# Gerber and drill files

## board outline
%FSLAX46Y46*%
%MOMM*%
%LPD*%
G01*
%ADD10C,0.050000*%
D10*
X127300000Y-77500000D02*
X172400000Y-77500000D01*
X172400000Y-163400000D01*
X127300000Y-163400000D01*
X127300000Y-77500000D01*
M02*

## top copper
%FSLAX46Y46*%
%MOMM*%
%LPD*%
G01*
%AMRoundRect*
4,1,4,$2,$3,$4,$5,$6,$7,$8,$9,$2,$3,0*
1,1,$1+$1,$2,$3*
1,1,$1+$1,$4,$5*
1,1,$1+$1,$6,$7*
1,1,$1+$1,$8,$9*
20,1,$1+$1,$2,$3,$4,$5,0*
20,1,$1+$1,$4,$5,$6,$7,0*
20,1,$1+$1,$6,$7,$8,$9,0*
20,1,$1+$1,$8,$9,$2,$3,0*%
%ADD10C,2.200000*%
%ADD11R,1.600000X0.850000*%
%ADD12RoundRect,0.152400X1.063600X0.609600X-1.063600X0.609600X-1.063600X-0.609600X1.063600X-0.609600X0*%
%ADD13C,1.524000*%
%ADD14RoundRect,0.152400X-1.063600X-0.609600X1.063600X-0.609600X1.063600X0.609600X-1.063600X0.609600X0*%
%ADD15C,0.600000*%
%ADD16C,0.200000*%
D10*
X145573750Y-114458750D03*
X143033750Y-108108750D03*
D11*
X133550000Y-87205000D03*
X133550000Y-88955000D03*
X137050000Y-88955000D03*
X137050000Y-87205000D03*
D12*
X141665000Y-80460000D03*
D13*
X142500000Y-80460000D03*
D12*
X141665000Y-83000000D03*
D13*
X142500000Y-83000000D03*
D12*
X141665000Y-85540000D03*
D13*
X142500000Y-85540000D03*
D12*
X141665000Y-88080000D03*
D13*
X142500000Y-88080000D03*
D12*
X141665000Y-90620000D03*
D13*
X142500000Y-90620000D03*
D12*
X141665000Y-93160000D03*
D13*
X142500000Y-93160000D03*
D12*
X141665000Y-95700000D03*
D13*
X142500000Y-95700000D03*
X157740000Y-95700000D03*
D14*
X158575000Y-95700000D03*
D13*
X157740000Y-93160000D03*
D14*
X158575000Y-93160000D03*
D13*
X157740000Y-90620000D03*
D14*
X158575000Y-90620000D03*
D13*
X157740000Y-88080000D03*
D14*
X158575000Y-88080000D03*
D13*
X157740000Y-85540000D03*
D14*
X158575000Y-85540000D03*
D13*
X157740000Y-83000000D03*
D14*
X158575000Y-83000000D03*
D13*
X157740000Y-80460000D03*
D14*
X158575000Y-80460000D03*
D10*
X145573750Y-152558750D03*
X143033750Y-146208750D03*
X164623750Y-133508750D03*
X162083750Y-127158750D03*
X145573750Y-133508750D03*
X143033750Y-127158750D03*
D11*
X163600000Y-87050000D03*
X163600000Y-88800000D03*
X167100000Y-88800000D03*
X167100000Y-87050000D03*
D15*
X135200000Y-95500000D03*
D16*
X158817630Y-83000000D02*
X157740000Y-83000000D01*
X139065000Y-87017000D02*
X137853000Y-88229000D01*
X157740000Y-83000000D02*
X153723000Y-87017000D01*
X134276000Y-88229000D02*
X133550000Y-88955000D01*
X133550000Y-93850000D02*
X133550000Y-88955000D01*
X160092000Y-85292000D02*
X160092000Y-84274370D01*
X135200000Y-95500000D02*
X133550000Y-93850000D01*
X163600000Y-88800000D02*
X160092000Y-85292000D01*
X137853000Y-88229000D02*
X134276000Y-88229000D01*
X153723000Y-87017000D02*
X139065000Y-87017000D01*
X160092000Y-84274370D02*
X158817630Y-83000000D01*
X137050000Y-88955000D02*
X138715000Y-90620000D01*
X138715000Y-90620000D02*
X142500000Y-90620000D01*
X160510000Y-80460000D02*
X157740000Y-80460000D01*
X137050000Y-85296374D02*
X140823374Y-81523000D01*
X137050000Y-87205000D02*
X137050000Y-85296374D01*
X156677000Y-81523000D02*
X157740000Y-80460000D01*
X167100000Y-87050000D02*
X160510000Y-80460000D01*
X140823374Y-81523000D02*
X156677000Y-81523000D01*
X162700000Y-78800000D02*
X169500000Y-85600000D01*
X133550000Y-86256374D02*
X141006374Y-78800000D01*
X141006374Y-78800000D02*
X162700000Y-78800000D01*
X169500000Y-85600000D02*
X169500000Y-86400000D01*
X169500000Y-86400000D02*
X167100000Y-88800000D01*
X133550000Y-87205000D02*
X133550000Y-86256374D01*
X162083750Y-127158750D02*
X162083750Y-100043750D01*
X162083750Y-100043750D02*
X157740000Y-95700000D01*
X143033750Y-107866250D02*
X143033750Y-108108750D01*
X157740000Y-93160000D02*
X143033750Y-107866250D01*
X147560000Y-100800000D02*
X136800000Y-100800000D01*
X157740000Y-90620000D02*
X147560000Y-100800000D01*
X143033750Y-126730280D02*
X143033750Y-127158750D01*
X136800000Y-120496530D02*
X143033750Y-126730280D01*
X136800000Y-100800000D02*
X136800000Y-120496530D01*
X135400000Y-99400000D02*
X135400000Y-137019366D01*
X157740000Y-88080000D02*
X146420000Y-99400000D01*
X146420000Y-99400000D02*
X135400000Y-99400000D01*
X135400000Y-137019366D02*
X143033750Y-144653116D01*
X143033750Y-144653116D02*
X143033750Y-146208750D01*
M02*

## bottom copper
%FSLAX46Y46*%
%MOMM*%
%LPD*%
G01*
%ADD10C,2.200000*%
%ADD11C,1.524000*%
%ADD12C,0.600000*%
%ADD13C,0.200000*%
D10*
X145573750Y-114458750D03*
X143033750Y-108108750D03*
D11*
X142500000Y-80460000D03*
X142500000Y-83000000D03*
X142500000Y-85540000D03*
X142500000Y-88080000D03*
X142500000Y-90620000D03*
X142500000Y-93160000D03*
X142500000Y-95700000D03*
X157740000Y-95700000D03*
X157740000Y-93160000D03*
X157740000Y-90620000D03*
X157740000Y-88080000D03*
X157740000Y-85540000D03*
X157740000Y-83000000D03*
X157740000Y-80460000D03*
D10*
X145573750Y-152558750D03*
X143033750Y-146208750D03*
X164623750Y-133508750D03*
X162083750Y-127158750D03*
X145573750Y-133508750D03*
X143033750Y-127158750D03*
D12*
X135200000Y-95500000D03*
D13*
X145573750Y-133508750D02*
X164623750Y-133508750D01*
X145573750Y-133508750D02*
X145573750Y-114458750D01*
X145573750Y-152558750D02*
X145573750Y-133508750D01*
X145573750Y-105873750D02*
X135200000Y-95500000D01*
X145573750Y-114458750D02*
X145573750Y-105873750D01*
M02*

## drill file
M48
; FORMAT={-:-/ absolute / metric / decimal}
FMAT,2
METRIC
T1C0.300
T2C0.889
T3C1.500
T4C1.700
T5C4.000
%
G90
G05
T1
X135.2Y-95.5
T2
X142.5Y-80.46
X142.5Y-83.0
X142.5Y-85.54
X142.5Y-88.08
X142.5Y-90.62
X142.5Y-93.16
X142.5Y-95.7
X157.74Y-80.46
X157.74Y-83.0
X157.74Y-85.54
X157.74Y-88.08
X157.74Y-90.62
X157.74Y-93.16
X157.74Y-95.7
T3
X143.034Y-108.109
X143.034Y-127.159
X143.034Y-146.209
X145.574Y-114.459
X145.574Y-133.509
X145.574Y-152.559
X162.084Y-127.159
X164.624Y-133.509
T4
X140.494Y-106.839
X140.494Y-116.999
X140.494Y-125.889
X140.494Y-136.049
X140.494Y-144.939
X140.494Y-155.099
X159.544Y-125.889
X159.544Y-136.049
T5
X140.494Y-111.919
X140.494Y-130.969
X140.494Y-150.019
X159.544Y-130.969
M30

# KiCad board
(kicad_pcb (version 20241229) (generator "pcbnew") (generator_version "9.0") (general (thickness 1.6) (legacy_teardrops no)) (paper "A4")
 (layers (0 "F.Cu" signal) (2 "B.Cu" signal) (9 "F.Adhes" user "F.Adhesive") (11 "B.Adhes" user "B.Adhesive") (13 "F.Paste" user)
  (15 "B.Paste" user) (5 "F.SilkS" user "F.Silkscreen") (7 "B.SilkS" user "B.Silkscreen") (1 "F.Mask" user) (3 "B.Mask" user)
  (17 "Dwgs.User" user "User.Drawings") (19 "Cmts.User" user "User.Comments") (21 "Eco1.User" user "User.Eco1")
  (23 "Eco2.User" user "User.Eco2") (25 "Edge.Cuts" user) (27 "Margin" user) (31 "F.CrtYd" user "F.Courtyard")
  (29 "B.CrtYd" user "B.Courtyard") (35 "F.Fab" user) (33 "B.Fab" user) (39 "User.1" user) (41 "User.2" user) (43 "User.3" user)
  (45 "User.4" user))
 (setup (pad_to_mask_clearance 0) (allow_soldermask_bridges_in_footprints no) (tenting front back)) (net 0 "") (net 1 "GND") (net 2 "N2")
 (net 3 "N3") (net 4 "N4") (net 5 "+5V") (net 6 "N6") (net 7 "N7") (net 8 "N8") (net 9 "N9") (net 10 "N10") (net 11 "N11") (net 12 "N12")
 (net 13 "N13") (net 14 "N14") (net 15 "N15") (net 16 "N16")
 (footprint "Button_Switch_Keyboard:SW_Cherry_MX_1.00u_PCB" (layer "F.Cu") (at 145.57375 114.45875 -90)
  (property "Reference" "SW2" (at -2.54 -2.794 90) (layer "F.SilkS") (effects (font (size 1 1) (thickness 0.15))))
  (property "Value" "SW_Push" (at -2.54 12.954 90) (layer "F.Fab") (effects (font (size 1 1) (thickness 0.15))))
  (pad "" np_thru_hole circle (at -7.62 5.08 270) (size 1.7 1.7) (drill 1.7) (layers "*.Cu" "*.Mask"))
  (pad "" np_thru_hole circle (at -2.54 5.08 270) (size 4 4) (drill 4) (layers "*.Cu" "*.Mask"))
  (pad "" np_thru_hole circle (at 2.54 5.08 270) (size 1.7 1.7) (drill 1.7) (layers "*.Cu" "*.Mask"))
  (pad "1" thru_hole circle (at 0 0 270) (size 2.2 2.2) (drill 1.5) (layers "*.Cu" "*.Mask") (remove_unused_layers no) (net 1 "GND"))
  (pad "2" thru_hole circle (at -6.35 2.54 270) (size 2.2 2.2) (drill 1.5) (layers "*.Cu" "*.Mask") (remove_unused_layers no) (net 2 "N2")))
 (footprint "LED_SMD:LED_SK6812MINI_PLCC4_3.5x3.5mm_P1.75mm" (layer "F.Cu") (at 135.3 88.08)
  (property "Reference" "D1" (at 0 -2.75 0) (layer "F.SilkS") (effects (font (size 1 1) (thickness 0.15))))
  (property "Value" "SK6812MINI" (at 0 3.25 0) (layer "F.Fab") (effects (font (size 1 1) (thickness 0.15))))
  (pad "1" smd rect (at -1.75 -0.875) (size 1.6 0.85) (layers "F.Cu" "F.Mask" "F.Paste") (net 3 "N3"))
  (pad "2" smd rect (at -1.75 0.875) (size 1.6 0.85) (layers "F.Cu" "F.Mask" "F.Paste") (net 1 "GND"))
  (pad "3" smd rect (at 1.75 0.875) (size 1.6 0.85) (layers "F.Cu" "F.Mask" "F.Paste") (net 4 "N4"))
  (pad "4" smd rect (at 1.75 -0.875) (size 1.6 0.85) (layers "F.Cu" "F.Mask" "F.Paste") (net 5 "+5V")))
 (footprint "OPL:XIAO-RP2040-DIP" (layer "F.Cu") (at 150.12 88.08)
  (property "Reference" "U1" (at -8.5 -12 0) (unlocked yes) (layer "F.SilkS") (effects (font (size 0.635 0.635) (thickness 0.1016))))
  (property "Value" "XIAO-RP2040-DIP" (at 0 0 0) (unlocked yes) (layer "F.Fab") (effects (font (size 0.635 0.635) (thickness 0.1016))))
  (pad "1" smd roundrect (at -8.455 -7.62 180) (size 2.432 1.524) (layers "F.Cu" "F.Mask") (roundrect_rratio 0.1) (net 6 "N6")
   (thermal_bridge_angle 45))
  (pad "1" thru_hole circle (at -7.62 -7.62 180) (size 1.524 1.524) (drill 0.889) (layers "*.Cu" "*.Mask") (remove_unused_layers no)
   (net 6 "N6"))
  (pad "2" smd roundrect (at -8.455 -5.08 180) (size 2.432 1.524) (layers "F.Cu" "F.Mask") (roundrect_rratio 0.1) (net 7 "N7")
   (thermal_bridge_angle 45))
  (pad "2" thru_hole circle (at -7.62 -5.08 180) (size 1.524 1.524) (drill 0.889) (layers "*.Cu" "*.Mask") (remove_unused_layers no)
   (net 7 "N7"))
  (pad "3" smd roundrect (at -8.455 -2.54 180) (size 2.432 1.524) (layers "F.Cu" "F.Mask") (roundrect_rratio 0.1) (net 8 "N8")
   (thermal_bridge_angle 45))
  (pad "3" thru_hole circle (at -7.62 -2.54 180) (size 1.524 1.524) (drill 0.889) (layers "*.Cu" "*.Mask") (remove_unused_layers no)
   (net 8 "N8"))
  (pad "4" smd roundrect (at -8.455 0 180) (size 2.432 1.524) (layers "F.Cu" "F.Mask") (roundrect_rratio 0.1) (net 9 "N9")
   (thermal_bridge_angle 45))
  (pad "4" thru_hole circle (at -7.62 0 180) (size 1.524 1.524) (drill 0.889) (layers "*.Cu" "*.Mask") (remove_unused_layers no)
   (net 9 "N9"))
  (pad "5" smd roundrect (at -8.455 2.54 180) (size 2.432 1.524) (layers "F.Cu" "F.Mask") (roundrect_rratio 0.1) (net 4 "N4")
   (thermal_bridge_angle 45))
  (pad "5" thru_hole circle (at -7.62 2.54 180) (size 1.524 1.524) (drill 0.889) (layers "*.Cu" "*.Mask") (remove_unused_layers no)
   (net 4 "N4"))
  (pad "6" smd roundrect (at -8.455 5.08 180) (size 2.432 1.524) (layers "F.Cu" "F.Mask") (roundrect_rratio 0.1) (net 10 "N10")
   (thermal_bridge_angle 45))
  (pad "6" thru_hole circle (at -7.62 5.08 180) (size 1.524 1.524) (drill 0.889) (layers "*.Cu" "*.Mask") (remove_unused_layers no)
   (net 10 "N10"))
  (pad "7" smd roundrect (at -8.455 7.62 180) (size 2.432 1.524) (layers "F.Cu" "F.Mask") (roundrect_rratio 0.1) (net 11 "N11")
   (thermal_bridge_angle 45))
  (pad "7" thru_hole circle (at -7.62 7.62 180) (size 1.524 1.524) (drill 0.889) (layers "*.Cu" "*.Mask") (remove_unused_layers no)
   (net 11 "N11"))
  (pad "8" thru_hole circle (at 7.62 7.62) (size 1.524 1.524) (drill 0.889) (layers "*.Cu" "*.Mask") (remove_unused_layers no)
   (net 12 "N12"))
  (pad "8" smd roundrect (at 8.455 7.62) (size 2.432 1.524) (layers "F.Cu" "F.Mask") (roundrect_rratio 0.1) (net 12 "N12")
   (thermal_bridge_angle 45))
  (pad "9" thru_hole circle (at 7.62 5.08) (size 1.524 1.524) (drill 0.889) (layers "*.Cu" "*.Mask") (remove_unused_layers no) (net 2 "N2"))
  (pad "9" smd roundrect (at 8.455 5.08) (size 2.432 1.524) (layers "F.Cu" "F.Mask") (roundrect_rratio 0.1) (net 2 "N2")
   (thermal_bridge_angle 45))
  (pad "10" thru_hole circle (at 7.62 2.54) (size 1.524 1.524) (drill 0.889) (layers "*.Cu" "*.Mask") (remove_unused_layers no)
   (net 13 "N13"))
  (pad "10" smd roundrect (at 8.455 2.54) (size 2.432 1.524) (layers "F.Cu" "F.Mask") (roundrect_rratio 0.1) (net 13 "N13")
   (thermal_bridge_angle 45))
  (pad "11" thru_hole circle (at 7.62 0) (size 1.524 1.524) (drill 0.889) (layers "*.Cu" "*.Mask") (remove_unused_layers no) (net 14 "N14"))
  (pad "11" smd roundrect (at 8.455 0) (size 2.432 1.524) (layers "F.Cu" "F.Mask") (roundrect_rratio 0.1) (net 14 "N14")
   (thermal_bridge_angle 45))
  (pad "12" thru_hole circle (at 7.62 -2.54) (size 1.524 1.524) (drill 0.889) (layers "*.Cu" "*.Mask") (remove_unused_layers no)
   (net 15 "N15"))
  (pad "12" smd roundrect (at 8.455 -2.54) (size 2.432 1.524) (layers "F.Cu" "F.Mask") (roundrect_rratio 0.1) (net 15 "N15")
   (thermal_bridge_angle 45))
  (pad "13" thru_hole circle (at 7.62 -5.08) (size 1.524 1.524) (drill 0.889) (layers "*.Cu" "*.Mask") (remove_unused_layers no)
   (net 1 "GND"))
  (pad "13" smd roundrect (at 8.455 -5.08) (size 2.432 1.524) (layers "F.Cu" "F.Mask") (roundrect_rratio 0.1) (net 1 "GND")
   (thermal_bridge_angle 45))
  (pad "14" thru_hole circle (at 7.62 -7.62) (size 1.524 1.524) (drill 0.889) (layers "*.Cu" "*.Mask") (remove_unused_layers no)
   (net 5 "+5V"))
  (pad "14" smd roundrect (at 8.455 -7.62) (size 2.432 1.524) (layers "F.Cu" "F.Mask") (roundrect_rratio 0.1) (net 5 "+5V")
   (thermal_bridge_angle 45)))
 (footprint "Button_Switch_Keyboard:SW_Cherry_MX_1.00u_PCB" (layer "F.Cu") (at 145.57375 152.55875 -90)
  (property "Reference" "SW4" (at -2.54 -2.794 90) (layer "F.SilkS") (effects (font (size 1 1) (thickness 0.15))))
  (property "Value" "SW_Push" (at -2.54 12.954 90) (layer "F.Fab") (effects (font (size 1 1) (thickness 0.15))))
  (pad "" np_thru_hole circle (at -7.62 5.08 270) (size 1.7 1.7) (drill 1.7) (layers "*.Cu" "*.Mask"))
  (pad "" np_thru_hole circle (at -2.54 5.08 270) (size 4 4) (drill 4) (layers "*.Cu" "*.Mask"))
  (pad "" np_thru_hole circle (at 2.54 5.08 270) (size 1.7 1.7) (drill 1.7) (layers "*.Cu" "*.Mask"))
  (pad "1" thru_hole circle (at 0 0 270) (size 2.2 2.2) (drill 1.5) (layers "*.Cu" "*.Mask") (remove_unused_layers no) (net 1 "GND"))
  (pad "2" thru_hole circle (at -6.35 2.54 270) (size 2.2 2.2) (drill 1.5) (layers "*.Cu" "*.Mask") (remove_unused_layers no) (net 14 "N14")))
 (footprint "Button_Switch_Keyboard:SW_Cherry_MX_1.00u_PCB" (layer "F.Cu") (at 164.62375 133.50875 -90)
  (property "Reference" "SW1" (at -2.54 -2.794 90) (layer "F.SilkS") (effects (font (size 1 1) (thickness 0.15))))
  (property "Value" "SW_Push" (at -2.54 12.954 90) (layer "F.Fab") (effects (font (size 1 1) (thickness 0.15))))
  (pad "" np_thru_hole circle (at -7.62 5.08 270) (size 1.7 1.7) (drill 1.7) (layers "*.Cu" "*.Mask"))
  (pad "" np_thru_hole circle (at -2.54 5.08 270) (size 4 4) (drill 4) (layers "*.Cu" "*.Mask"))
  (pad "" np_thru_hole circle (at 2.54 5.08 270) (size 1.7 1.7) (drill 1.7) (layers "*.Cu" "*.Mask"))
  (pad "1" thru_hole circle (at 0 0 270) (size 2.2 2.2) (drill 1.5) (layers "*.Cu" "*.Mask") (remove_unused_layers no) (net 1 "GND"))
  (pad "2" thru_hole circle (at -6.35 2.54 270) (size 2.2 2.2) (drill 1.5) (layers "*.Cu" "*.Mask") (remove_unused_layers no) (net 12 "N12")))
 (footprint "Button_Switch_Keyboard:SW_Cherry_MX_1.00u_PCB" (layer "F.Cu") (at 145.57375 133.50875 -90)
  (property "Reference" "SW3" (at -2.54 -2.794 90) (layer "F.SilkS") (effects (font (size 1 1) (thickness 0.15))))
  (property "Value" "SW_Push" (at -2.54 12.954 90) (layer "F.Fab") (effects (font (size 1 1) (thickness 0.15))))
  (pad "" np_thru_hole circle (at -7.62 5.08 270) (size 1.7 1.7) (drill 1.7) (layers "*.Cu" "*.Mask"))
  (pad "" np_thru_hole circle (at -2.54 5.08 270) (size 4 4) (drill 4) (layers "*.Cu" "*.Mask"))
  (pad "" np_thru_hole circle (at 2.54 5.08 270) (size 1.7 1.7) (drill 1.7) (layers "*.Cu" "*.Mask"))
  (pad "1" thru_hole circle (at 0 0 270) (size 2.2 2.2) (drill 1.5) (layers "*.Cu" "*.Mask") (remove_unused_layers no) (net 1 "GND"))
  (pad "2" thru_hole circle (at -6.35 2.54 270) (size 2.2 2.2) (drill 1.5) (layers "*.Cu" "*.Mask") (remove_unused_layers no) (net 13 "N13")))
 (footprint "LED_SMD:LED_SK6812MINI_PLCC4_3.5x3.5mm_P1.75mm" (layer "F.Cu") (at 165.35 87.925)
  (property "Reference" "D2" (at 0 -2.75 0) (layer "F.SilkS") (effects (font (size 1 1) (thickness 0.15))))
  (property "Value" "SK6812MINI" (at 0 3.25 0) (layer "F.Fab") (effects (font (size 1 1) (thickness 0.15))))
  (pad "1" smd rect (at -1.75 -0.875) (size 1.6 0.85) (layers "F.Cu" "F.Mask" "F.Paste") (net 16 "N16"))
  (pad "2" smd rect (at -1.75 0.875) (size 1.6 0.85) (layers "F.Cu" "F.Mask" "F.Paste") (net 1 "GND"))
  (pad "3" smd rect (at 1.75 0.875) (size 1.6 0.85) (layers "F.Cu" "F.Mask" "F.Paste") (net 3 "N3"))
  (pad "4" smd rect (at 1.75 -0.875) (size 1.6 0.85) (layers "F.Cu" "F.Mask" "F.Paste") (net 5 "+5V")))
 (gr_rect (start 127.3 77.5) (end 172.4 163.4) (stroke (width 0.05) (type default)) (fill no) (layer "Edge.Cuts"))
 (segment (start 158.81763 83) (end 157.74 83) (width 0.2) (layer "F.Cu") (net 1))
 (segment (start 139.065 87.017) (end 137.853 88.229) (width 0.2) (layer "F.Cu") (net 1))
 (segment (start 157.74 83) (end 153.723 87.017) (width 0.2) (layer "F.Cu") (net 1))
 (segment (start 134.276 88.229) (end 133.55 88.955) (width 0.2) (layer "F.Cu") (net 1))
 (segment (start 133.55 93.85) (end 133.55 88.955) (width 0.2) (layer "F.Cu") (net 1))
 (segment (start 160.092 85.292) (end 160.092 84.27437) (width 0.2) (layer "F.Cu") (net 1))
 (segment (start 135.2 95.5) (end 133.55 93.85) (width 0.2) (layer "F.Cu") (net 1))
 (segment (start 163.6 88.8) (end 160.092 85.292) (width 0.2) (layer "F.Cu") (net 1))
 (segment (start 137.853 88.229) (end 134.276 88.229) (width 0.2) (layer "F.Cu") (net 1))
 (segment (start 153.723 87.017) (end 139.065 87.017) (width 0.2) (layer "F.Cu") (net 1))
 (segment (start 160.092 84.27437) (end 158.81763 83) (width 0.2) (layer "F.Cu") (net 1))
 (via (at 135.2 95.5) (size 0.6) (drill 0.3) (layers "F.Cu" "B.Cu") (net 1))
 (segment (start 145.57375 133.50875) (end 164.62375 133.50875) (width 0.2) (layer "B.Cu") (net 1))
 (segment (start 145.57375 133.50875) (end 145.57375 114.45875) (width 0.2) (layer "B.Cu") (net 1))
 (segment (start 145.57375 152.55875) (end 145.57375 133.50875) (width 0.2) (layer "B.Cu") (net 1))
 (segment (start 145.57375 105.87375) (end 135.2 95.5) (width 0.2) (layer "B.Cu") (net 1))
 (segment (start 145.57375 114.45875) (end 145.57375 105.87375) (width 0.2) (layer "B.Cu") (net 1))
 (segment (start 137.05 88.955) (end 138.715 90.62) (width 0.2) (layer "F.Cu") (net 4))
 (segment (start 138.715 90.62) (end 142.5 90.62) (width 0.2) (layer "F.Cu") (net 4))
 (segment (start 160.51 80.46) (end 157.74 80.46) (width 0.2) (layer "F.Cu") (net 5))
 (segment (start 137.05 85.296374) (end 140.823374 81.523) (width 0.2) (layer "F.Cu") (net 5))
 (segment (start 137.05 87.205) (end 137.05 85.296374) (width 0.2) (layer "F.Cu") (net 5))
 (segment (start 156.677 81.523) (end 157.74 80.46) (width 0.2) (layer "F.Cu") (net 5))
 (segment (start 167.1 87.05) (end 160.51 80.46) (width 0.2) (layer "F.Cu") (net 5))
 (segment (start 140.823374 81.523) (end 156.677 81.523) (width 0.2) (layer "F.Cu") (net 5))
 (segment (start 162.7 78.8) (end 169.5 85.6) (width 0.2) (layer "F.Cu") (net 3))
 (segment (start 133.55 86.256374) (end 141.006374 78.8) (width 0.2) (layer "F.Cu") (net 3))
 (segment (start 141.006374 78.8) (end 162.7 78.8) (width 0.2) (layer "F.Cu") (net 3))
 (segment (start 169.5 85.6) (end 169.5 86.4) (width 0.2) (layer "F.Cu") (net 3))
 (segment (start 169.5 86.4) (end 167.1 88.8) (width 0.2) (layer "F.Cu") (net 3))
 (segment (start 133.55 87.205) (end 133.55 86.256374) (width 0.2) (layer "F.Cu") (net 3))
 (segment (start 162.08375 127.15875) (end 162.08375 100.04375) (width 0.2) (layer "F.Cu") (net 12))
 (segment (start 162.08375 100.04375) (end 157.74 95.7) (width 0.2) (layer "F.Cu") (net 12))
 (segment (start 143.03375 107.86625) (end 143.03375 108.10875) (width 0.2) (layer "F.Cu") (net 2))
 (segment (start 157.74 93.16) (end 143.03375 107.86625) (width 0.2) (layer "F.Cu") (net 2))
 (segment (start 147.56 100.8) (end 136.8 100.8) (width 0.2) (layer "F.Cu") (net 13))
 (segment (start 157.74 90.62) (end 147.56 100.8) (width 0.2) (layer "F.Cu") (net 13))
 (segment (start 143.03375 126.73028) (end 143.03375 127.15875) (width 0.2) (layer "F.Cu") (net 13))
 (segment (start 136.8 120.49653) (end 143.03375 126.73028) (width 0.2) (layer "F.Cu") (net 13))
 (segment (start 136.8 100.8) (end 136.8 120.49653) (width 0.2) (layer "F.Cu") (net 13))
 (segment (start 135.4 99.4) (end 135.4 137.019366) (width 0.2) (layer "F.Cu") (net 14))
 (segment (start 157.74 88.08) (end 146.42 99.4) (width 0.2) (layer "F.Cu") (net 14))
 (segment (start 146.42 99.4) (end 135.4 99.4) (width 0.2) (layer "F.Cu") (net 14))
 (segment (start 135.4 137.019366) (end 143.03375 144.653116) (width 0.2) (layer "F.Cu") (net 14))
 (segment (start 143.03375 144.653116) (end 143.03375 146.20875) (width 0.2) (layer "F.Cu") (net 14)))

